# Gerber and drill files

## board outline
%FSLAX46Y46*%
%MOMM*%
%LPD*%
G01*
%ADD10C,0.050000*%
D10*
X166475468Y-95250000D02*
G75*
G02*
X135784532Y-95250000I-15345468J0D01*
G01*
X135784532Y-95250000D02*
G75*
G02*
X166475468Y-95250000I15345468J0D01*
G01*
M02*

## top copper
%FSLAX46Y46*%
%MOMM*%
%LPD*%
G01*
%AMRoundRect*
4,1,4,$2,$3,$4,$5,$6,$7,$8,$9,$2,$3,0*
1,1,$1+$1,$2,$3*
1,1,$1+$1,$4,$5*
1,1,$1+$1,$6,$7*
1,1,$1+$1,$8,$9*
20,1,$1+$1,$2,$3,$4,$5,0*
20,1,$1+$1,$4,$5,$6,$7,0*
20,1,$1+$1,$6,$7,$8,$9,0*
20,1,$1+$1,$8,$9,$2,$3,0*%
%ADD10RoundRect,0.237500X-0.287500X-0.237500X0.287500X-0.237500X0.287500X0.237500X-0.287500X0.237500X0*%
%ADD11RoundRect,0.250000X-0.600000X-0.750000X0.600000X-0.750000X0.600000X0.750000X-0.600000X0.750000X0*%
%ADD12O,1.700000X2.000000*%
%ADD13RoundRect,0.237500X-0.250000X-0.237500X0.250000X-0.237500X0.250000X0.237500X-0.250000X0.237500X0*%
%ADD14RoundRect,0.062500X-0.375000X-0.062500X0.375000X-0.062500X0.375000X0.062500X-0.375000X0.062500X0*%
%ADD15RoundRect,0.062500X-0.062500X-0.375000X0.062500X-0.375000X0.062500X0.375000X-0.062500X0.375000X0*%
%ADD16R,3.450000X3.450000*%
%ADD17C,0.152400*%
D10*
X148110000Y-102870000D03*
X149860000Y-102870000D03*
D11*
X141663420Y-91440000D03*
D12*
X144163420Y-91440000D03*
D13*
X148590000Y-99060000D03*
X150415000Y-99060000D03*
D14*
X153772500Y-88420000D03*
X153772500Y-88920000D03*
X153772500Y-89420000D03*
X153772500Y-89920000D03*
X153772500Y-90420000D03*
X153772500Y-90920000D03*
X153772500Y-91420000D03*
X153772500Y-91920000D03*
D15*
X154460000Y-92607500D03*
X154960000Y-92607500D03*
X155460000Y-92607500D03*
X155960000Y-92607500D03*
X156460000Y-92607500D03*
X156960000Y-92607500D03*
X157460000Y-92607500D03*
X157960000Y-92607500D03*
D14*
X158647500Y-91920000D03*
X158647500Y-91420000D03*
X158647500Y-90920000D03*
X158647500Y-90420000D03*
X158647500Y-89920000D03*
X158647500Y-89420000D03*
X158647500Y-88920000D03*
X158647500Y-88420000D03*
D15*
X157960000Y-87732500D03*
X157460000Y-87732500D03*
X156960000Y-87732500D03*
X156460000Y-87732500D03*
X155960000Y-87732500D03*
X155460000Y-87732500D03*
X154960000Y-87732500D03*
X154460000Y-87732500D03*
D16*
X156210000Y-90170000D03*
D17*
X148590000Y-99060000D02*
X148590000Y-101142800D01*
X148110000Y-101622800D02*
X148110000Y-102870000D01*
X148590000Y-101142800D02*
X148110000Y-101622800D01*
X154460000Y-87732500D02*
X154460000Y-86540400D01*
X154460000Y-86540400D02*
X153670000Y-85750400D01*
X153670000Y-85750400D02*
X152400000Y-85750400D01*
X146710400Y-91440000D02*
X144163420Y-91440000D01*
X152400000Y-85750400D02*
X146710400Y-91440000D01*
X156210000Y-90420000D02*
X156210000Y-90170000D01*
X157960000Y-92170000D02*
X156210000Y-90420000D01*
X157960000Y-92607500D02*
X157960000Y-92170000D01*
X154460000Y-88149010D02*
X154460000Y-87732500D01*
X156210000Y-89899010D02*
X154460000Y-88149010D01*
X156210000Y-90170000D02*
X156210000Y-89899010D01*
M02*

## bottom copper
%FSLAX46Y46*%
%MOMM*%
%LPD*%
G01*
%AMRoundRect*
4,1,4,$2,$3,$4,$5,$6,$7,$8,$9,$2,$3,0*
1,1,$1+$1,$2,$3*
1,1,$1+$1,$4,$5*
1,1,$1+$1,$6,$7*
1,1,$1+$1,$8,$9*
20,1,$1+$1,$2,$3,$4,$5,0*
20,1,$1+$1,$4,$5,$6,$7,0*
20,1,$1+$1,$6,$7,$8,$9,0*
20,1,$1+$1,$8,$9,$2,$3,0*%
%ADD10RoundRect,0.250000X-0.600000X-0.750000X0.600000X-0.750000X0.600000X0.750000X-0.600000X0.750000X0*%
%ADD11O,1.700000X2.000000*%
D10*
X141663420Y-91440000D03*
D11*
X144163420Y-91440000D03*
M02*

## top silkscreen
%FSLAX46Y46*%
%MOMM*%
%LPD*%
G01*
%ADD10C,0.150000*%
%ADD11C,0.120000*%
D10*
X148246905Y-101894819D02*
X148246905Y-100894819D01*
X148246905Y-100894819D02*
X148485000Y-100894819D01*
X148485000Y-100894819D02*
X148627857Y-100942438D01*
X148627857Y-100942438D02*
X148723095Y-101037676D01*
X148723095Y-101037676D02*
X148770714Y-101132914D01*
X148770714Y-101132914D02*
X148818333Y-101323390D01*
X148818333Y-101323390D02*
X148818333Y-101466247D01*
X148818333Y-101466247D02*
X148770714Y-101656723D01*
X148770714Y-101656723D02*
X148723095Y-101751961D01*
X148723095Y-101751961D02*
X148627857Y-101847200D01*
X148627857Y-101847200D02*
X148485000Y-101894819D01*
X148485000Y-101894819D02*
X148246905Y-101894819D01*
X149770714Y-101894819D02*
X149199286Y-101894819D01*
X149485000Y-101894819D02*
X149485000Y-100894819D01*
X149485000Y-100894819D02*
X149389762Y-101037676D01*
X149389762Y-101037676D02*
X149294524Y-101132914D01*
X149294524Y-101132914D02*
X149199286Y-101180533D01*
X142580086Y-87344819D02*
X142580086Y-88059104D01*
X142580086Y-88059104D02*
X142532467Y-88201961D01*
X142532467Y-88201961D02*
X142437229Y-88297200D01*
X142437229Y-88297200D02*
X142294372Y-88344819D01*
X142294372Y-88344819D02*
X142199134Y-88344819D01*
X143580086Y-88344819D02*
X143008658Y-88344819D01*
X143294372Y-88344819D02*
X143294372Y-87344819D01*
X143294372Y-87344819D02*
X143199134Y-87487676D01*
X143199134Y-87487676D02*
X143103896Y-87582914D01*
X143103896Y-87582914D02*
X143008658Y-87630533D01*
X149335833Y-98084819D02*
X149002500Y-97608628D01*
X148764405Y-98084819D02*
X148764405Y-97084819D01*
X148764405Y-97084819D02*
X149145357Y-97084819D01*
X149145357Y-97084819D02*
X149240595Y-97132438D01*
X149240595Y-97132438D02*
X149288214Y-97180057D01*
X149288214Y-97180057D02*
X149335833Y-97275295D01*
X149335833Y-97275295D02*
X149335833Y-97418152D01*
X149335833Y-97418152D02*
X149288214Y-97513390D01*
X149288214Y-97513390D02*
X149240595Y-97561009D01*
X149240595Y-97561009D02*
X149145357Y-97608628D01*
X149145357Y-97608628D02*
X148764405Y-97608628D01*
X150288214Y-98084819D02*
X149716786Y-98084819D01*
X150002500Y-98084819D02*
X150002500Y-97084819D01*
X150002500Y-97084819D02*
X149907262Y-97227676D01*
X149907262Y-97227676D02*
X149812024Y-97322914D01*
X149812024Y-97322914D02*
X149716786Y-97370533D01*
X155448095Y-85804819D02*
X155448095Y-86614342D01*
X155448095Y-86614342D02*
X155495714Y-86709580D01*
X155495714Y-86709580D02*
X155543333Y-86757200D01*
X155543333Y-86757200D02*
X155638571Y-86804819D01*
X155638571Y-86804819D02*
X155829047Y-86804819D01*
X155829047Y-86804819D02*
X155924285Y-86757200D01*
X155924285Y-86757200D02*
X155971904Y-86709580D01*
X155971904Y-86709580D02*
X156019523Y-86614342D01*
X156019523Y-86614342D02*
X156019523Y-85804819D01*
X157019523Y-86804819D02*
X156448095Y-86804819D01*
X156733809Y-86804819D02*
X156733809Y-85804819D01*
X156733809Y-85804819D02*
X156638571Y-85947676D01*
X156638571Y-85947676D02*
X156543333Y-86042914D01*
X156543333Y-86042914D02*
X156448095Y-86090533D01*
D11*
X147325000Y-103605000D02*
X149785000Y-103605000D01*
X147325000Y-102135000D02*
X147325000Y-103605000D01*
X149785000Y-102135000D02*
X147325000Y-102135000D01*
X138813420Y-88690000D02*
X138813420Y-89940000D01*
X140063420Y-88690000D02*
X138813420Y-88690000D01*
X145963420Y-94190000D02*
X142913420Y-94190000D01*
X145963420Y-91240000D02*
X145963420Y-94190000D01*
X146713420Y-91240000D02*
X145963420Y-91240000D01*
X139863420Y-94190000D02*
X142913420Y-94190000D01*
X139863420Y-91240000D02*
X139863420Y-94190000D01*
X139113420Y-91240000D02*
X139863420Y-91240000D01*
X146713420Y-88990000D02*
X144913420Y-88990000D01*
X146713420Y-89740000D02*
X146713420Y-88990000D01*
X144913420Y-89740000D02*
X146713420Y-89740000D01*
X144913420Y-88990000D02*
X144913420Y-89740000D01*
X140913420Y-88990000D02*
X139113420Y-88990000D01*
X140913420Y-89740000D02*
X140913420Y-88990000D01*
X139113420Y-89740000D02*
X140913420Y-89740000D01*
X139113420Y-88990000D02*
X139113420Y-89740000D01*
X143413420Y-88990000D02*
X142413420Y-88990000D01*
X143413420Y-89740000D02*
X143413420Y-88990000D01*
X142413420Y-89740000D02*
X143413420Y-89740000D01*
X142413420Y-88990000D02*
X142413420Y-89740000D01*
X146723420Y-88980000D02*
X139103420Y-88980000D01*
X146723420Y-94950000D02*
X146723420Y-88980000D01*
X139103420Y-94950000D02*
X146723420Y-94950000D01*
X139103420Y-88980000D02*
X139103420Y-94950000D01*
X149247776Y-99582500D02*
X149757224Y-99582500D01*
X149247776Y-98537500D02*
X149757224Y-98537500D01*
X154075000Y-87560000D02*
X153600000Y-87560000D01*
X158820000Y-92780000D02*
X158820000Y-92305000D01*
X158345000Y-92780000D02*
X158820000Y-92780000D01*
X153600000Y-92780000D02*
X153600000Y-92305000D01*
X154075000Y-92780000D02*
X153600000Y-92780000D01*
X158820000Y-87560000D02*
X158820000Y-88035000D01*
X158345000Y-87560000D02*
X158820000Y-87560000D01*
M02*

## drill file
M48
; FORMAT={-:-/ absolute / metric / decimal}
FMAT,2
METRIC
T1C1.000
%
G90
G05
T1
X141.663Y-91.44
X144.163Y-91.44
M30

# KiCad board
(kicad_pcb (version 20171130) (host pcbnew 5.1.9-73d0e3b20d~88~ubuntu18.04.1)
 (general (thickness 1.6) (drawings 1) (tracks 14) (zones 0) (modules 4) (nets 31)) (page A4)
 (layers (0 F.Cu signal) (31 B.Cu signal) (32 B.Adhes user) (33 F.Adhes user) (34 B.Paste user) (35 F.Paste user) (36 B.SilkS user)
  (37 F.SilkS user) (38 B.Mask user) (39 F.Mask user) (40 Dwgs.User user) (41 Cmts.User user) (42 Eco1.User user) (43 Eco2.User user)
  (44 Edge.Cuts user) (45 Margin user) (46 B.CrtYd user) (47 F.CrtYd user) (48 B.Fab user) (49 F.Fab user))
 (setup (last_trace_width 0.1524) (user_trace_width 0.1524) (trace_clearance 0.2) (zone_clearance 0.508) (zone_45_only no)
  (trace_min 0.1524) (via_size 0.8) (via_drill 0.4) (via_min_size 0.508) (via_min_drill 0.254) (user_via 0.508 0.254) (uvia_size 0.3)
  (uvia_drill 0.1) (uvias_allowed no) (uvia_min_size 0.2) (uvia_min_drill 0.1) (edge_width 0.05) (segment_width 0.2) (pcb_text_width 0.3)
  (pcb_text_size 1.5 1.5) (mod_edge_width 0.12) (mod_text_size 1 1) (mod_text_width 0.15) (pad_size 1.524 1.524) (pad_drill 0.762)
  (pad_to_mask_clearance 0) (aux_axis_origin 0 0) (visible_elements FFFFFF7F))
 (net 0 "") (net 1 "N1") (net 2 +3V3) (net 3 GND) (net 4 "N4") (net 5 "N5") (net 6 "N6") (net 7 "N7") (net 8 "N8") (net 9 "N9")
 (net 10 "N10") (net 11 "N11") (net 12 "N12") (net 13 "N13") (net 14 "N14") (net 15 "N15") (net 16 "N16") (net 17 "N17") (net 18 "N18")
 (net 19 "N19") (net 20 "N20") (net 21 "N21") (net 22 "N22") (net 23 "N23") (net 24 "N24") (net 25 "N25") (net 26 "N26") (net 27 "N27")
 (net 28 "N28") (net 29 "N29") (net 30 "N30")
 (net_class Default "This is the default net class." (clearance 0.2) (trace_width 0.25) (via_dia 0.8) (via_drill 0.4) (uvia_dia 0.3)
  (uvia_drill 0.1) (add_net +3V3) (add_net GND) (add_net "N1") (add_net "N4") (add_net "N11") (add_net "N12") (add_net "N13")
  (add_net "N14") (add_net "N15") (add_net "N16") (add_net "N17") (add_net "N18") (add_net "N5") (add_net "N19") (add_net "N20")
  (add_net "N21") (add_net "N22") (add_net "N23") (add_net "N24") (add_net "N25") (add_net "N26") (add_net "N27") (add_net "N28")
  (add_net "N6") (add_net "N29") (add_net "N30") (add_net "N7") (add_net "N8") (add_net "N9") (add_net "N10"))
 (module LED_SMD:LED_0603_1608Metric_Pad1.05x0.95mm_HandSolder (layer F.Cu) (at 148.985 102.87)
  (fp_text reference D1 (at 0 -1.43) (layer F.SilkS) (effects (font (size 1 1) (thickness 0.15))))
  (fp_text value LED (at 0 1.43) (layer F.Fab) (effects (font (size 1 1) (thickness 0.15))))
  (fp_line (start -1.66 0.735) (end 0.8 0.735) (layer F.SilkS) (width 0.12))
  (fp_line (start -1.66 -0.735) (end -1.66 0.735) (layer F.SilkS) (width 0.12))
  (fp_line (start 0.8 -0.735) (end -1.66 -0.735) (layer F.SilkS) (width 0.12))
  (pad 1 smd roundrect (at -0.875 0) (size 1.05 0.95) (layers F.Cu F.Paste F.Mask) (roundrect_rratio 0.25) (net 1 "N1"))
  (pad 2 smd roundrect (at 0.875 0) (size 1.05 0.95) (layers F.Cu F.Paste F.Mask) (roundrect_rratio 0.25) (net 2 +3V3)))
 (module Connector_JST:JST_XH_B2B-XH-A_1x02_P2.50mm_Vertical (layer F.Cu) (at 141.66342 91.44)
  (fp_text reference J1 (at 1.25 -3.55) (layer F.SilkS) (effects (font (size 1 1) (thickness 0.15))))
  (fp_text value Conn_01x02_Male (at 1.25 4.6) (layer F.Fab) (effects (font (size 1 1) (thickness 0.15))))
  (fp_line (start -2.85 -2.75) (end -2.85 -1.5) (layer F.SilkS) (width 0.12))
  (fp_line (start -1.6 -2.75) (end -2.85 -2.75) (layer F.SilkS) (width 0.12))
  (fp_line (start 4.3 2.75) (end 1.25 2.75) (layer F.SilkS) (width 0.12))
  (fp_line (start 4.3 -0.2) (end 4.3 2.75) (layer F.SilkS) (width 0.12))
  (fp_line (start 5.05 -0.2) (end 4.3 -0.2) (layer F.SilkS) (width 0.12))
  (fp_line (start -1.8 2.75) (end 1.25 2.75) (layer F.SilkS) (width 0.12))
  (fp_line (start -1.8 -0.2) (end -1.8 2.75) (layer F.SilkS) (width 0.12))
  (fp_line (start -2.55 -0.2) (end -1.8 -0.2) (layer F.SilkS) (width 0.12))
  (fp_line (start 5.05 -2.45) (end 3.25 -2.45) (layer F.SilkS) (width 0.12))
  (fp_line (start 5.05 -1.7) (end 5.05 -2.45) (layer F.SilkS) (width 0.12))
  (fp_line (start 3.25 -1.7) (end 5.05 -1.7) (layer F.SilkS) (width 0.12))
  (fp_line (start 3.25 -2.45) (end 3.25 -1.7) (layer F.SilkS) (width 0.12))
  (fp_line (start -0.75 -2.45) (end -2.55 -2.45) (layer F.SilkS) (width 0.12))
  (fp_line (start -0.75 -1.7) (end -0.75 -2.45) (layer F.SilkS) (width 0.12))
  (fp_line (start -2.55 -1.7) (end -0.75 -1.7) (layer F.SilkS) (width 0.12))
  (fp_line (start -2.55 -2.45) (end -2.55 -1.7) (layer F.SilkS) (width 0.12))
  (fp_line (start 1.75 -2.45) (end 0.75 -2.45) (layer F.SilkS) (width 0.12))
  (fp_line (start 1.75 -1.7) (end 1.75 -2.45) (layer F.SilkS) (width 0.12))
  (fp_line (start 0.75 -1.7) (end 1.75 -1.7) (layer F.SilkS) (width 0.12))
  (fp_line (start 0.75 -2.45) (end 0.75 -1.7) (layer F.SilkS) (width 0.12))
  (fp_line (start 5.06 -2.46) (end -2.56 -2.46) (layer F.SilkS) (width 0.12))
  (fp_line (start 5.06 3.51) (end 5.06 -2.46) (layer F.SilkS) (width 0.12))
  (fp_line (start -2.56 3.51) (end 5.06 3.51) (layer F.SilkS) (width 0.12))
  (fp_line (start -2.56 -2.46) (end -2.56 3.51) (layer F.SilkS) (width 0.12))
  (pad 1 thru_hole roundrect (at 0 0) (size 1.7 2) (drill 1) (layers *.Cu *.Mask) (roundrect_rratio 0.147059) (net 2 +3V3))
  (pad 2 thru_hole oval (at 2.5 0) (size 1.7 2) (drill 1) (layers *.Cu *.Mask) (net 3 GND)))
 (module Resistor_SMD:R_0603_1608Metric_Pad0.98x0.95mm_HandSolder (layer F.Cu) (at 149.5025 99.06)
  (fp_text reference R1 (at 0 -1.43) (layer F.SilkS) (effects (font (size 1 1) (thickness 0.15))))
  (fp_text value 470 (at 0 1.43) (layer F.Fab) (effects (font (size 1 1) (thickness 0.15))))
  (fp_line (start -0.254724 0.5225) (end 0.254724 0.5225) (layer F.SilkS) (width 0.12))
  (fp_line (start -0.254724 -0.5225) (end 0.254724 -0.5225) (layer F.SilkS) (width 0.12))
  (pad 1 smd roundrect (at -0.9125 0) (size 0.975 0.95) (layers F.Cu F.Paste F.Mask) (roundrect_rratio 0.25) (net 1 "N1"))
  (pad 2 smd roundrect (at 0.9125 0) (size 0.975 0.95) (layers F.Cu F.Paste F.Mask) (roundrect_rratio 0.25) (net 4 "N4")))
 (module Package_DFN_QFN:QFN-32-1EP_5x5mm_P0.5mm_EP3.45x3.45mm (layer F.Cu) (at 156.21 90.17)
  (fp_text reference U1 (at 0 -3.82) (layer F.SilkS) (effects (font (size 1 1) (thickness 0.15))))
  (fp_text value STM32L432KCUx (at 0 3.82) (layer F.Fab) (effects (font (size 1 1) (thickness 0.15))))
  (fp_line (start -2.135 -2.61) (end -2.61 -2.61) (layer F.SilkS) (width 0.12))
  (fp_line (start 2.61 2.61) (end 2.61 2.135) (layer F.SilkS) (width 0.12))
  (fp_line (start 2.135 2.61) (end 2.61 2.61) (layer F.SilkS) (width 0.12))
  (fp_line (start -2.61 2.61) (end -2.61 2.135) (layer F.SilkS) (width 0.12))
  (fp_line (start -2.135 2.61) (end -2.61 2.61) (layer F.SilkS) (width 0.12))
  (fp_line (start 2.61 -2.61) (end 2.61 -2.135) (layer F.SilkS) (width 0.12))
  (fp_line (start 2.135 -2.61) (end 2.61 -2.61) (layer F.SilkS) (width 0.12))
  (pad 1 smd roundrect (at -2.4375 -1.75) (size 0.875 0.25) (layers F.Cu F.Paste F.Mask) (roundrect_rratio 0.25) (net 2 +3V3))
  (pad 2 smd roundrect (at -2.4375 -1.25) (size 0.875 0.25) (layers F.Cu F.Paste F.Mask) (roundrect_rratio 0.25) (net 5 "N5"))
  (pad 3 smd roundrect (at -2.4375 -0.75) (size 0.875 0.25) (layers F.Cu F.Paste F.Mask) (roundrect_rratio 0.25) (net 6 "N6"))
  (pad 4 smd roundrect (at -2.4375 -0.25) (size 0.875 0.25) (layers F.Cu F.Paste F.Mask) (roundrect_rratio 0.25) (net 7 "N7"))
  (pad 5 smd roundrect (at -2.4375 0.25) (size 0.875 0.25) (layers F.Cu F.Paste F.Mask) (roundrect_rratio 0.25) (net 2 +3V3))
  (pad 6 smd roundrect (at -2.4375 0.75) (size 0.875 0.25) (layers F.Cu F.Paste F.Mask) (roundrect_rratio 0.25) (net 4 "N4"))
  (pad 7 smd roundrect (at -2.4375 1.25) (size 0.875 0.25) (layers F.Cu F.Paste F.Mask) (roundrect_rratio 0.25) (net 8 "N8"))
  (pad 8 smd roundrect (at -2.4375 1.75) (size 0.875 0.25) (layers F.Cu F.Paste F.Mask) (roundrect_rratio 0.25) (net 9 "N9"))
  (pad 9 smd roundrect (at -1.75 2.4375) (size 0.25 0.875) (layers F.Cu F.Paste F.Mask) (roundrect_rratio 0.25) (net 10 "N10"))
  (pad 10 smd roundrect (at -1.25 2.4375) (size 0.25 0.875) (layers F.Cu F.Paste F.Mask) (roundrect_rratio 0.25) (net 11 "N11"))
  (pad 11 smd roundrect (at -0.75 2.4375) (size 0.25 0.875) (layers F.Cu F.Paste F.Mask) (roundrect_rratio 0.25) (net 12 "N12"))
  (pad 12 smd roundrect (at -0.25 2.4375) (size 0.25 0.875) (layers F.Cu F.Paste F.Mask) (roundrect_rratio 0.25) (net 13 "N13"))
  (pad 13 smd roundrect (at 0.25 2.4375) (size 0.25 0.875) (layers F.Cu F.Paste F.Mask) (roundrect_rratio 0.25) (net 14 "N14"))
  (pad 14 smd roundrect (at 0.75 2.4375) (size 0.25 0.875) (layers F.Cu F.Paste F.Mask) (roundrect_rratio 0.25) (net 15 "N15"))
  (pad 15 smd roundrect (at 1.25 2.4375) (size 0.25 0.875) (layers F.Cu F.Paste F.Mask) (roundrect_rratio 0.25) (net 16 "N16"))
  (pad 16 smd roundrect (at 1.75 2.4375) (size 0.25 0.875) (layers F.Cu F.Paste F.Mask) (roundrect_rratio 0.25) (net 3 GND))
  (pad 17 smd roundrect (at 2.4375 1.75) (size 0.875 0.25) (layers F.Cu F.Paste F.Mask) (roundrect_rratio 0.25) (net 2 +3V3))
  (pad 18 smd roundrect (at 2.4375 1.25) (size 0.875 0.25) (layers F.Cu F.Paste F.Mask) (roundrect_rratio 0.25) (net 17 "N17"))
  (pad 19 smd roundrect (at 2.4375 0.75) (size 0.875 0.25) (layers F.Cu F.Paste F.Mask) (roundrect_rratio 0.25) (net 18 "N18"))
  (pad 20 smd roundrect (at 2.4375 0.25) (size 0.875 0.25) (layers F.Cu F.Paste F.Mask) (roundrect_rratio 0.25) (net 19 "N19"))
  (pad 21 smd roundrect (at 2.4375 -0.25) (size 0.875 0.25) (layers F.Cu F.Paste F.Mask) (roundrect_rratio 0.25) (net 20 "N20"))
  (pad 22 smd roundrect (at 2.4375 -0.75) (size 0.875 0.25) (layers F.Cu F.Paste F.Mask) (roundrect_rratio 0.25) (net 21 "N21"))
  (pad 23 smd roundrect (at 2.4375 -1.25) (size 0.875 0.25) (layers F.Cu F.Paste F.Mask) (roundrect_rratio 0.25) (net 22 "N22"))
  (pad 24 smd roundrect (at 2.4375 -1.75) (size 0.875 0.25) (layers F.Cu F.Paste F.Mask) (roundrect_rratio 0.25) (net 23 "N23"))
  (pad 25 smd roundrect (at 1.75 -2.4375) (size 0.25 0.875) (layers F.Cu F.Paste F.Mask) (roundrect_rratio 0.25) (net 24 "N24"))
  (pad 26 smd roundrect (at 1.25 -2.4375) (size 0.25 0.875) (layers F.Cu F.Paste F.Mask) (roundrect_rratio 0.25) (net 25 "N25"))
  (pad 27 smd roundrect (at 0.75 -2.4375) (size 0.25 0.875) (layers F.Cu F.Paste F.Mask) (roundrect_rratio 0.25) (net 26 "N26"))
  (pad 28 smd roundrect (at 0.25 -2.4375) (size 0.25 0.875) (layers F.Cu F.Paste F.Mask) (roundrect_rratio 0.25) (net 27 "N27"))
  (pad 29 smd roundrect (at -0.25 -2.4375) (size 0.25 0.875) (layers F.Cu F.Paste F.Mask) (roundrect_rratio 0.25) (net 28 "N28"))
  (pad 30 smd roundrect (at -0.75 -2.4375) (size 0.25 0.875) (layers F.Cu F.Paste F.Mask) (roundrect_rratio 0.25) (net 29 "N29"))
  (pad 31 smd roundrect (at -1.25 -2.4375) (size 0.25 0.875) (layers F.Cu F.Paste F.Mask) (roundrect_rratio 0.25) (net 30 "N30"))
  (pad 32 smd roundrect (at -1.75 -2.4375) (size 0.25 0.875) (layers F.Cu F.Paste F.Mask) (roundrect_rratio 0.25) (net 3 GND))
  (pad 33 smd rect (at 0 0) (size 3.45 3.45) (layers F.Cu F.Mask) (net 3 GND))
  (pad "" smd roundrect (at -1.15 -1.15) (size 0.93 0.93) (layers F.Paste) (roundrect_rratio 0.25))
  (pad "" smd roundrect (at -1.15 0) (size 0.93 0.93) (layers F.Paste) (roundrect_rratio 0.25))
  (pad "" smd roundrect (at -1.15 1.15) (size 0.93 0.93) (layers F.Paste) (roundrect_rratio 0.25))
  (pad "" smd roundrect (at 0 -1.15) (size 0.93 0.93) (layers F.Paste) (roundrect_rratio 0.25))
  (pad "" smd roundrect (at 0 0) (size 0.93 0.93) (layers F.Paste) (roundrect_rratio 0.25))
  (pad "" smd roundrect (at 0 1.15) (size 0.93 0.93) (layers F.Paste) (roundrect_rratio 0.25))
  (pad "" smd roundrect (at 1.15 -1.15) (size 0.93 0.93) (layers F.Paste) (roundrect_rratio 0.25))
  (pad "" smd roundrect (at 1.15 0) (size 0.93 0.93) (layers F.Paste) (roundrect_rratio 0.25))
  (pad "" smd roundrect (at 1.15 1.15) (size 0.93 0.93) (layers F.Paste) (roundrect_rratio 0.25)))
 (gr_circle (center 151.13 95.25) (end 137.16 88.9) (layer Edge.Cuts) (width 0.05))
 (segment (start 148.59 99.06) (end 148.59 101.1428) (width 0.1524) (layer F.Cu) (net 1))
 (segment (start 148.11 101.6228) (end 148.11 102.87) (width 0.1524) (layer F.Cu) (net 1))
 (segment (start 148.59 101.1428) (end 148.11 101.6228) (width 0.1524) (layer F.Cu) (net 1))
 (segment (start 154.46 87.7325) (end 154.46 86.5404) (width 0.1524) (layer F.Cu) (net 3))
 (segment (start 154.46 86.5404) (end 153.67 85.7504) (width 0.1524) (layer F.Cu) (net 3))
 (segment (start 153.67 85.7504) (end 152.4 85.7504) (width 0.1524) (layer F.Cu) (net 3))
 (segment (start 146.7104 91.44) (end 144.16342 91.44) (width 0.1524) (layer F.Cu) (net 3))
 (segment (start 152.4 85.7504) (end 146.7104 91.44) (width 0.1524) (layer F.Cu) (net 3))
 (segment (start 156.21 90.42) (end 156.21 90.17) (width 0.1524) (layer F.Cu) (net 3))
 (segment (start 157.96 92.17) (end 156.21 90.42) (width 0.1524) (layer F.Cu) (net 3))
 (segment (start 157.96 92.6075) (end 157.96 92.17) (width 0.1524) (layer F.Cu) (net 3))
 (segment (start 154.46 88.14901) (end 154.46 87.7325) (width 0.1524) (layer F.Cu) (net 3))
 (segment (start 156.21 89.89901) (end 154.46 88.14901) (width 0.1524) (layer F.Cu) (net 3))
 (segment (start 156.21 90.17) (end 156.21 89.89901) (width 0.1524) (layer F.Cu) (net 3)))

